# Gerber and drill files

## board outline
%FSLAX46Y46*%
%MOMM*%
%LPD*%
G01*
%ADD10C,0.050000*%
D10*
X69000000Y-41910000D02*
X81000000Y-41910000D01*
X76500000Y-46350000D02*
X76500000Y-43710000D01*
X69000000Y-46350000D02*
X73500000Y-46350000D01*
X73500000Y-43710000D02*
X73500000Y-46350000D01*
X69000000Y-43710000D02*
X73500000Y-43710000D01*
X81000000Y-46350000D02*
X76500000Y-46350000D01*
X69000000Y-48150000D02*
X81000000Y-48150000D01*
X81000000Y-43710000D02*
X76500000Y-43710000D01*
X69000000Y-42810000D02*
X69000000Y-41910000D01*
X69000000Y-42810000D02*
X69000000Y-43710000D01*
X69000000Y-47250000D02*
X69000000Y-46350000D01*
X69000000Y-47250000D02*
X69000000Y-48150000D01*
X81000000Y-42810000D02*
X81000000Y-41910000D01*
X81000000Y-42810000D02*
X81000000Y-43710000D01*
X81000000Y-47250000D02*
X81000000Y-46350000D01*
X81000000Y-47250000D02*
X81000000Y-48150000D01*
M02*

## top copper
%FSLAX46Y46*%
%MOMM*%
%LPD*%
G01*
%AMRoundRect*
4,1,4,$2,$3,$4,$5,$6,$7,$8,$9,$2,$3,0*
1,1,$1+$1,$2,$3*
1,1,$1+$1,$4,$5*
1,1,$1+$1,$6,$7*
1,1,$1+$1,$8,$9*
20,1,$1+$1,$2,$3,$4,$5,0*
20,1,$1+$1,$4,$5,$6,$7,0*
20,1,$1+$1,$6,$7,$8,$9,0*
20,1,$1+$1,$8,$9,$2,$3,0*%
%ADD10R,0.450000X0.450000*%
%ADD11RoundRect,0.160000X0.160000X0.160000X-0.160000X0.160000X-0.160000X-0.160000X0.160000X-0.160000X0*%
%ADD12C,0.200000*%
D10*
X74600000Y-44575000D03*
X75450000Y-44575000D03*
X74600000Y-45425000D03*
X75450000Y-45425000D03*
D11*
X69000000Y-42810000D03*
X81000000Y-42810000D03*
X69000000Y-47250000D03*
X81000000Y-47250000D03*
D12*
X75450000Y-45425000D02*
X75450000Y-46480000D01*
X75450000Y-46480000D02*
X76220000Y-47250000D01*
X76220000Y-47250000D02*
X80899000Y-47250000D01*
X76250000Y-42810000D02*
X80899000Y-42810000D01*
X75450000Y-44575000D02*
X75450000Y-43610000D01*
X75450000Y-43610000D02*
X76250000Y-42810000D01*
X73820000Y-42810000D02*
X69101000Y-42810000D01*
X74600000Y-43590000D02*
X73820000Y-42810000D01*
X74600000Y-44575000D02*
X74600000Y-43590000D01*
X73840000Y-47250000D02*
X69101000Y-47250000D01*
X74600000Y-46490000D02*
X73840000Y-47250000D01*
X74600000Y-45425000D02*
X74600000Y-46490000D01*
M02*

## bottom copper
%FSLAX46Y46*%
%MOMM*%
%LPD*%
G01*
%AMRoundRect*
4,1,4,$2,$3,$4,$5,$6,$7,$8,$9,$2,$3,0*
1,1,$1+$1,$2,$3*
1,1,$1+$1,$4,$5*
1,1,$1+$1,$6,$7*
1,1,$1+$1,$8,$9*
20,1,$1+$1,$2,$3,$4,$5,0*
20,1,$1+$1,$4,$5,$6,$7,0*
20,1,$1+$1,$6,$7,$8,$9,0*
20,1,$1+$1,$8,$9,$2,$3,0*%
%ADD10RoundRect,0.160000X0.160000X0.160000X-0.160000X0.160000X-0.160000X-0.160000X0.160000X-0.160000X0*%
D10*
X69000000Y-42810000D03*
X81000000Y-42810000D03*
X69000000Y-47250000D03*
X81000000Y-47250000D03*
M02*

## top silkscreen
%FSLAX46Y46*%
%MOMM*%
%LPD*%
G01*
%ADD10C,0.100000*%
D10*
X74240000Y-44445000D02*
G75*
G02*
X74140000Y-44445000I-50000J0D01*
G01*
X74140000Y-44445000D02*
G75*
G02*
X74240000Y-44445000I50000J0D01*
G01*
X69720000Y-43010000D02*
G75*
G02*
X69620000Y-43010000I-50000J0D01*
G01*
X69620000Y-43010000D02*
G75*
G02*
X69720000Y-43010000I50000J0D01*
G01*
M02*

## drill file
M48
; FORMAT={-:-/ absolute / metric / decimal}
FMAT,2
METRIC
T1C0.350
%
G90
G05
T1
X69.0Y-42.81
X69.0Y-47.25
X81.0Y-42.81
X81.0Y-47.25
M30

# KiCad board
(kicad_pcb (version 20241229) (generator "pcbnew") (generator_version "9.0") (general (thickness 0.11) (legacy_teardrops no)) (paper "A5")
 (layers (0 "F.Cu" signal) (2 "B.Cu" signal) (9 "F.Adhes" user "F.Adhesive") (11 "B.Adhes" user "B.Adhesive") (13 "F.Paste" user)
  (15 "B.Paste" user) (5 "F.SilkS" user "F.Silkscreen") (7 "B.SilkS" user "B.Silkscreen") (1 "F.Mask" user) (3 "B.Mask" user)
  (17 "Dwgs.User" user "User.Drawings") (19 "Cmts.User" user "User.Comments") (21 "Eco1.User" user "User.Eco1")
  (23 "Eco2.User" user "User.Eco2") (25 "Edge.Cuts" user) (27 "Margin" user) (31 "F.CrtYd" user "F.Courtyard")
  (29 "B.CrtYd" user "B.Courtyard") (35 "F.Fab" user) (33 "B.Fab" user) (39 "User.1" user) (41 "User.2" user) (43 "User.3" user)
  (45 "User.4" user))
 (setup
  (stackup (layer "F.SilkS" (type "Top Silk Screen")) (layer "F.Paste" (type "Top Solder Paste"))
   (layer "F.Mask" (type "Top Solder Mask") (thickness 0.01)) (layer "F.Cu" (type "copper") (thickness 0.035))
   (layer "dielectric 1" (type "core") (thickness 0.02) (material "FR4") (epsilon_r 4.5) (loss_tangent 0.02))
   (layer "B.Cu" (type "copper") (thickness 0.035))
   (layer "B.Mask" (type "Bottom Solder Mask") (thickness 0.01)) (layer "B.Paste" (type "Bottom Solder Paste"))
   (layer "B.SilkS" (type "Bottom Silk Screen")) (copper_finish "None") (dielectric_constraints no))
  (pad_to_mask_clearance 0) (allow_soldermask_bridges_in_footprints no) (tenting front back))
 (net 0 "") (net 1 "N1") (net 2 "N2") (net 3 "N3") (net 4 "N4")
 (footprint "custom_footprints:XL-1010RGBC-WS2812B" (layer "F.Cu") (at 75 45.025)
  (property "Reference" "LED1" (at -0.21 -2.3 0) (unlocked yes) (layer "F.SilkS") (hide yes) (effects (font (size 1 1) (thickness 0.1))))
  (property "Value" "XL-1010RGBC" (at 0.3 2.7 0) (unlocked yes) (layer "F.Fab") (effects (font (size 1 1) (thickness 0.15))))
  (fp_circle (center -0.81 -0.58) (end -0.76 -0.58) (stroke (width 0.1) (type default)) (fill no) (layer "F.SilkS"))
  (pad "1" smd rect (at -0.4 -0.45 90) (size 0.45 0.45) (layers "F.Cu" "F.Mask" "F.Paste") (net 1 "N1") (thermal_bridge_angle 45))
  (pad "2" smd rect (at 0.45 -0.45 90) (size 0.45 0.45) (layers "F.Cu" "F.Mask" "F.Paste") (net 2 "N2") (thermal_bridge_angle 45))
  (pad "3" smd rect (at -0.4 0.4 90) (size 0.45 0.45) (layers "F.Cu" "F.Mask" "F.Paste") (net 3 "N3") (thermal_bridge_angle 45))
  (pad "4" smd rect (at 0.45 0.4 90) (size 0.45 0.45) (layers "F.Cu" "F.Mask" "F.Paste") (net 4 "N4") (thermal_bridge_angle 45)))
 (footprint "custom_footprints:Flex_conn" (layer "F.Cu") (at 75 45)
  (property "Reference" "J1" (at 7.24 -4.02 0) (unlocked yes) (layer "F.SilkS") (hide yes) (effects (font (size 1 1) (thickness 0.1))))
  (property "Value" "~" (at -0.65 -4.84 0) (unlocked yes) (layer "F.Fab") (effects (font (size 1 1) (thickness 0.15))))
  (fp_circle (center -5.33 -1.99) (end -5.28 -1.99) (stroke (width 0.1) (type default)) (fill no) (layer "F.SilkS"))
  (fp_line (start -6 -2.19) (end -6 -3.09) (stroke (width 0.05) (type default)) (layer "Edge.Cuts"))
  (fp_line (start -6 -2.19) (end -6 -1.29) (stroke (width 0.05) (type default)) (layer "Edge.Cuts"))
  (fp_line (start -6 2.25) (end -6 1.35) (stroke (width 0.05) (type default)) (layer "Edge.Cuts"))
  (fp_line (start -6 2.25) (end -6 3.15) (stroke (width 0.05) (type default)) (layer "Edge.Cuts"))
  (fp_line (start 6 -2.19) (end 6 -3.09) (stroke (width 0.05) (type default)) (layer "Edge.Cuts"))
  (fp_line (start 6 -2.19) (end 6 -1.29) (stroke (width 0.05) (type default)) (layer "Edge.Cuts"))
  (fp_line (start 6 2.25) (end 6 1.35) (stroke (width 0.05) (type default)) (layer "Edge.Cuts"))
  (fp_line (start 6 2.25) (end 6 3.15) (stroke (width 0.05) (type default)) (layer "Edge.Cuts"))
  (pad "1" thru_hole roundrect (at -6 -2.19 180) (size 0.64 0.64) (drill 0.35) (layers "*.Cu" "*.Mask") (remove_unused_layers no)
   (roundrect_rratio 0.25) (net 1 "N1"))
  (pad "2" thru_hole roundrect (at 6 -2.19 180) (size 0.64 0.64) (drill 0.35) (layers "*.Cu" "*.Mask") (remove_unused_layers no)
   (roundrect_rratio 0.25) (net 2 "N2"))
  (pad "3" thru_hole roundrect (at -6 2.25 180) (size 0.64 0.64) (drill 0.35) (layers "*.Cu" "*.Mask") (remove_unused_layers no)
   (roundrect_rratio 0.25) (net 3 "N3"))
  (pad "4" thru_hole roundrect (at 6 2.25 180) (size 0.64 0.64) (drill 0.35) (layers "*.Cu" "*.Mask") (remove_unused_layers no)
   (roundrect_rratio 0.25) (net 4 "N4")))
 (gr_line (start 69 41.91) (end 81 41.91) (stroke (width 0.05) (type default)) (layer "Edge.Cuts"))
 (gr_line (start 76.5 46.35) (end 76.5 43.71) (stroke (width 0.05) (type default)) (layer "Edge.Cuts"))
 (gr_line (start 69 46.35) (end 73.5 46.35) (stroke (width 0.05) (type default)) (layer "Edge.Cuts"))
 (gr_line (start 73.5 43.71) (end 73.5 46.35) (stroke (width 0.05) (type default)) (layer "Edge.Cuts"))
 (gr_line (start 69 43.71) (end 73.5 43.71) (stroke (width 0.05) (type default)) (layer "Edge.Cuts"))
 (gr_line (start 81 46.35) (end 76.5 46.35) (stroke (width 0.05) (type default)) (layer "Edge.Cuts"))
 (gr_line (start 69 48.15) (end 81 48.15) (stroke (width 0.05) (type default)) (layer "Edge.Cuts"))
 (gr_line (start 81 43.71) (end 76.5 43.71) (stroke (width 0.05) (type default)) (layer "Edge.Cuts"))
 (segment (start 75.45 45.425) (end 75.45 46.48) (width 0.2) (layer "F.Cu") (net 4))
 (segment (start 75.45 46.48) (end 76.22 47.25) (width 0.2) (layer "F.Cu") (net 4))
 (segment (start 76.22 47.25) (end 80.899 47.25) (width 0.2) (layer "F.Cu") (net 4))
 (segment (start 76.25 42.81) (end 80.899 42.81) (width 0.2) (layer "F.Cu") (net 2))
 (segment (start 75.45 44.575) (end 75.45 43.61) (width 0.2) (layer "F.Cu") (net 2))
 (segment (start 75.45 43.61) (end 76.25 42.81) (width 0.2) (layer "F.Cu") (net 2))
 (segment (start 73.82 42.81) (end 69.101 42.81) (width 0.2) (layer "F.Cu") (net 1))
 (segment (start 74.6 43.59) (end 73.82 42.81) (width 0.2) (layer "F.Cu") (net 1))
 (segment (start 74.6 44.575) (end 74.6 43.59) (width 0.2) (layer "F.Cu") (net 1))
 (segment (start 73.84 47.25) (end 69.101 47.25) (width 0.2) (layer "F.Cu") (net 3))
 (segment (start 74.6 46.49) (end 73.84 47.25) (width 0.2) (layer "F.Cu") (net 3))
 (segment (start 74.6 45.425) (end 74.6 46.49) (width 0.2) (layer "F.Cu") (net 3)))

